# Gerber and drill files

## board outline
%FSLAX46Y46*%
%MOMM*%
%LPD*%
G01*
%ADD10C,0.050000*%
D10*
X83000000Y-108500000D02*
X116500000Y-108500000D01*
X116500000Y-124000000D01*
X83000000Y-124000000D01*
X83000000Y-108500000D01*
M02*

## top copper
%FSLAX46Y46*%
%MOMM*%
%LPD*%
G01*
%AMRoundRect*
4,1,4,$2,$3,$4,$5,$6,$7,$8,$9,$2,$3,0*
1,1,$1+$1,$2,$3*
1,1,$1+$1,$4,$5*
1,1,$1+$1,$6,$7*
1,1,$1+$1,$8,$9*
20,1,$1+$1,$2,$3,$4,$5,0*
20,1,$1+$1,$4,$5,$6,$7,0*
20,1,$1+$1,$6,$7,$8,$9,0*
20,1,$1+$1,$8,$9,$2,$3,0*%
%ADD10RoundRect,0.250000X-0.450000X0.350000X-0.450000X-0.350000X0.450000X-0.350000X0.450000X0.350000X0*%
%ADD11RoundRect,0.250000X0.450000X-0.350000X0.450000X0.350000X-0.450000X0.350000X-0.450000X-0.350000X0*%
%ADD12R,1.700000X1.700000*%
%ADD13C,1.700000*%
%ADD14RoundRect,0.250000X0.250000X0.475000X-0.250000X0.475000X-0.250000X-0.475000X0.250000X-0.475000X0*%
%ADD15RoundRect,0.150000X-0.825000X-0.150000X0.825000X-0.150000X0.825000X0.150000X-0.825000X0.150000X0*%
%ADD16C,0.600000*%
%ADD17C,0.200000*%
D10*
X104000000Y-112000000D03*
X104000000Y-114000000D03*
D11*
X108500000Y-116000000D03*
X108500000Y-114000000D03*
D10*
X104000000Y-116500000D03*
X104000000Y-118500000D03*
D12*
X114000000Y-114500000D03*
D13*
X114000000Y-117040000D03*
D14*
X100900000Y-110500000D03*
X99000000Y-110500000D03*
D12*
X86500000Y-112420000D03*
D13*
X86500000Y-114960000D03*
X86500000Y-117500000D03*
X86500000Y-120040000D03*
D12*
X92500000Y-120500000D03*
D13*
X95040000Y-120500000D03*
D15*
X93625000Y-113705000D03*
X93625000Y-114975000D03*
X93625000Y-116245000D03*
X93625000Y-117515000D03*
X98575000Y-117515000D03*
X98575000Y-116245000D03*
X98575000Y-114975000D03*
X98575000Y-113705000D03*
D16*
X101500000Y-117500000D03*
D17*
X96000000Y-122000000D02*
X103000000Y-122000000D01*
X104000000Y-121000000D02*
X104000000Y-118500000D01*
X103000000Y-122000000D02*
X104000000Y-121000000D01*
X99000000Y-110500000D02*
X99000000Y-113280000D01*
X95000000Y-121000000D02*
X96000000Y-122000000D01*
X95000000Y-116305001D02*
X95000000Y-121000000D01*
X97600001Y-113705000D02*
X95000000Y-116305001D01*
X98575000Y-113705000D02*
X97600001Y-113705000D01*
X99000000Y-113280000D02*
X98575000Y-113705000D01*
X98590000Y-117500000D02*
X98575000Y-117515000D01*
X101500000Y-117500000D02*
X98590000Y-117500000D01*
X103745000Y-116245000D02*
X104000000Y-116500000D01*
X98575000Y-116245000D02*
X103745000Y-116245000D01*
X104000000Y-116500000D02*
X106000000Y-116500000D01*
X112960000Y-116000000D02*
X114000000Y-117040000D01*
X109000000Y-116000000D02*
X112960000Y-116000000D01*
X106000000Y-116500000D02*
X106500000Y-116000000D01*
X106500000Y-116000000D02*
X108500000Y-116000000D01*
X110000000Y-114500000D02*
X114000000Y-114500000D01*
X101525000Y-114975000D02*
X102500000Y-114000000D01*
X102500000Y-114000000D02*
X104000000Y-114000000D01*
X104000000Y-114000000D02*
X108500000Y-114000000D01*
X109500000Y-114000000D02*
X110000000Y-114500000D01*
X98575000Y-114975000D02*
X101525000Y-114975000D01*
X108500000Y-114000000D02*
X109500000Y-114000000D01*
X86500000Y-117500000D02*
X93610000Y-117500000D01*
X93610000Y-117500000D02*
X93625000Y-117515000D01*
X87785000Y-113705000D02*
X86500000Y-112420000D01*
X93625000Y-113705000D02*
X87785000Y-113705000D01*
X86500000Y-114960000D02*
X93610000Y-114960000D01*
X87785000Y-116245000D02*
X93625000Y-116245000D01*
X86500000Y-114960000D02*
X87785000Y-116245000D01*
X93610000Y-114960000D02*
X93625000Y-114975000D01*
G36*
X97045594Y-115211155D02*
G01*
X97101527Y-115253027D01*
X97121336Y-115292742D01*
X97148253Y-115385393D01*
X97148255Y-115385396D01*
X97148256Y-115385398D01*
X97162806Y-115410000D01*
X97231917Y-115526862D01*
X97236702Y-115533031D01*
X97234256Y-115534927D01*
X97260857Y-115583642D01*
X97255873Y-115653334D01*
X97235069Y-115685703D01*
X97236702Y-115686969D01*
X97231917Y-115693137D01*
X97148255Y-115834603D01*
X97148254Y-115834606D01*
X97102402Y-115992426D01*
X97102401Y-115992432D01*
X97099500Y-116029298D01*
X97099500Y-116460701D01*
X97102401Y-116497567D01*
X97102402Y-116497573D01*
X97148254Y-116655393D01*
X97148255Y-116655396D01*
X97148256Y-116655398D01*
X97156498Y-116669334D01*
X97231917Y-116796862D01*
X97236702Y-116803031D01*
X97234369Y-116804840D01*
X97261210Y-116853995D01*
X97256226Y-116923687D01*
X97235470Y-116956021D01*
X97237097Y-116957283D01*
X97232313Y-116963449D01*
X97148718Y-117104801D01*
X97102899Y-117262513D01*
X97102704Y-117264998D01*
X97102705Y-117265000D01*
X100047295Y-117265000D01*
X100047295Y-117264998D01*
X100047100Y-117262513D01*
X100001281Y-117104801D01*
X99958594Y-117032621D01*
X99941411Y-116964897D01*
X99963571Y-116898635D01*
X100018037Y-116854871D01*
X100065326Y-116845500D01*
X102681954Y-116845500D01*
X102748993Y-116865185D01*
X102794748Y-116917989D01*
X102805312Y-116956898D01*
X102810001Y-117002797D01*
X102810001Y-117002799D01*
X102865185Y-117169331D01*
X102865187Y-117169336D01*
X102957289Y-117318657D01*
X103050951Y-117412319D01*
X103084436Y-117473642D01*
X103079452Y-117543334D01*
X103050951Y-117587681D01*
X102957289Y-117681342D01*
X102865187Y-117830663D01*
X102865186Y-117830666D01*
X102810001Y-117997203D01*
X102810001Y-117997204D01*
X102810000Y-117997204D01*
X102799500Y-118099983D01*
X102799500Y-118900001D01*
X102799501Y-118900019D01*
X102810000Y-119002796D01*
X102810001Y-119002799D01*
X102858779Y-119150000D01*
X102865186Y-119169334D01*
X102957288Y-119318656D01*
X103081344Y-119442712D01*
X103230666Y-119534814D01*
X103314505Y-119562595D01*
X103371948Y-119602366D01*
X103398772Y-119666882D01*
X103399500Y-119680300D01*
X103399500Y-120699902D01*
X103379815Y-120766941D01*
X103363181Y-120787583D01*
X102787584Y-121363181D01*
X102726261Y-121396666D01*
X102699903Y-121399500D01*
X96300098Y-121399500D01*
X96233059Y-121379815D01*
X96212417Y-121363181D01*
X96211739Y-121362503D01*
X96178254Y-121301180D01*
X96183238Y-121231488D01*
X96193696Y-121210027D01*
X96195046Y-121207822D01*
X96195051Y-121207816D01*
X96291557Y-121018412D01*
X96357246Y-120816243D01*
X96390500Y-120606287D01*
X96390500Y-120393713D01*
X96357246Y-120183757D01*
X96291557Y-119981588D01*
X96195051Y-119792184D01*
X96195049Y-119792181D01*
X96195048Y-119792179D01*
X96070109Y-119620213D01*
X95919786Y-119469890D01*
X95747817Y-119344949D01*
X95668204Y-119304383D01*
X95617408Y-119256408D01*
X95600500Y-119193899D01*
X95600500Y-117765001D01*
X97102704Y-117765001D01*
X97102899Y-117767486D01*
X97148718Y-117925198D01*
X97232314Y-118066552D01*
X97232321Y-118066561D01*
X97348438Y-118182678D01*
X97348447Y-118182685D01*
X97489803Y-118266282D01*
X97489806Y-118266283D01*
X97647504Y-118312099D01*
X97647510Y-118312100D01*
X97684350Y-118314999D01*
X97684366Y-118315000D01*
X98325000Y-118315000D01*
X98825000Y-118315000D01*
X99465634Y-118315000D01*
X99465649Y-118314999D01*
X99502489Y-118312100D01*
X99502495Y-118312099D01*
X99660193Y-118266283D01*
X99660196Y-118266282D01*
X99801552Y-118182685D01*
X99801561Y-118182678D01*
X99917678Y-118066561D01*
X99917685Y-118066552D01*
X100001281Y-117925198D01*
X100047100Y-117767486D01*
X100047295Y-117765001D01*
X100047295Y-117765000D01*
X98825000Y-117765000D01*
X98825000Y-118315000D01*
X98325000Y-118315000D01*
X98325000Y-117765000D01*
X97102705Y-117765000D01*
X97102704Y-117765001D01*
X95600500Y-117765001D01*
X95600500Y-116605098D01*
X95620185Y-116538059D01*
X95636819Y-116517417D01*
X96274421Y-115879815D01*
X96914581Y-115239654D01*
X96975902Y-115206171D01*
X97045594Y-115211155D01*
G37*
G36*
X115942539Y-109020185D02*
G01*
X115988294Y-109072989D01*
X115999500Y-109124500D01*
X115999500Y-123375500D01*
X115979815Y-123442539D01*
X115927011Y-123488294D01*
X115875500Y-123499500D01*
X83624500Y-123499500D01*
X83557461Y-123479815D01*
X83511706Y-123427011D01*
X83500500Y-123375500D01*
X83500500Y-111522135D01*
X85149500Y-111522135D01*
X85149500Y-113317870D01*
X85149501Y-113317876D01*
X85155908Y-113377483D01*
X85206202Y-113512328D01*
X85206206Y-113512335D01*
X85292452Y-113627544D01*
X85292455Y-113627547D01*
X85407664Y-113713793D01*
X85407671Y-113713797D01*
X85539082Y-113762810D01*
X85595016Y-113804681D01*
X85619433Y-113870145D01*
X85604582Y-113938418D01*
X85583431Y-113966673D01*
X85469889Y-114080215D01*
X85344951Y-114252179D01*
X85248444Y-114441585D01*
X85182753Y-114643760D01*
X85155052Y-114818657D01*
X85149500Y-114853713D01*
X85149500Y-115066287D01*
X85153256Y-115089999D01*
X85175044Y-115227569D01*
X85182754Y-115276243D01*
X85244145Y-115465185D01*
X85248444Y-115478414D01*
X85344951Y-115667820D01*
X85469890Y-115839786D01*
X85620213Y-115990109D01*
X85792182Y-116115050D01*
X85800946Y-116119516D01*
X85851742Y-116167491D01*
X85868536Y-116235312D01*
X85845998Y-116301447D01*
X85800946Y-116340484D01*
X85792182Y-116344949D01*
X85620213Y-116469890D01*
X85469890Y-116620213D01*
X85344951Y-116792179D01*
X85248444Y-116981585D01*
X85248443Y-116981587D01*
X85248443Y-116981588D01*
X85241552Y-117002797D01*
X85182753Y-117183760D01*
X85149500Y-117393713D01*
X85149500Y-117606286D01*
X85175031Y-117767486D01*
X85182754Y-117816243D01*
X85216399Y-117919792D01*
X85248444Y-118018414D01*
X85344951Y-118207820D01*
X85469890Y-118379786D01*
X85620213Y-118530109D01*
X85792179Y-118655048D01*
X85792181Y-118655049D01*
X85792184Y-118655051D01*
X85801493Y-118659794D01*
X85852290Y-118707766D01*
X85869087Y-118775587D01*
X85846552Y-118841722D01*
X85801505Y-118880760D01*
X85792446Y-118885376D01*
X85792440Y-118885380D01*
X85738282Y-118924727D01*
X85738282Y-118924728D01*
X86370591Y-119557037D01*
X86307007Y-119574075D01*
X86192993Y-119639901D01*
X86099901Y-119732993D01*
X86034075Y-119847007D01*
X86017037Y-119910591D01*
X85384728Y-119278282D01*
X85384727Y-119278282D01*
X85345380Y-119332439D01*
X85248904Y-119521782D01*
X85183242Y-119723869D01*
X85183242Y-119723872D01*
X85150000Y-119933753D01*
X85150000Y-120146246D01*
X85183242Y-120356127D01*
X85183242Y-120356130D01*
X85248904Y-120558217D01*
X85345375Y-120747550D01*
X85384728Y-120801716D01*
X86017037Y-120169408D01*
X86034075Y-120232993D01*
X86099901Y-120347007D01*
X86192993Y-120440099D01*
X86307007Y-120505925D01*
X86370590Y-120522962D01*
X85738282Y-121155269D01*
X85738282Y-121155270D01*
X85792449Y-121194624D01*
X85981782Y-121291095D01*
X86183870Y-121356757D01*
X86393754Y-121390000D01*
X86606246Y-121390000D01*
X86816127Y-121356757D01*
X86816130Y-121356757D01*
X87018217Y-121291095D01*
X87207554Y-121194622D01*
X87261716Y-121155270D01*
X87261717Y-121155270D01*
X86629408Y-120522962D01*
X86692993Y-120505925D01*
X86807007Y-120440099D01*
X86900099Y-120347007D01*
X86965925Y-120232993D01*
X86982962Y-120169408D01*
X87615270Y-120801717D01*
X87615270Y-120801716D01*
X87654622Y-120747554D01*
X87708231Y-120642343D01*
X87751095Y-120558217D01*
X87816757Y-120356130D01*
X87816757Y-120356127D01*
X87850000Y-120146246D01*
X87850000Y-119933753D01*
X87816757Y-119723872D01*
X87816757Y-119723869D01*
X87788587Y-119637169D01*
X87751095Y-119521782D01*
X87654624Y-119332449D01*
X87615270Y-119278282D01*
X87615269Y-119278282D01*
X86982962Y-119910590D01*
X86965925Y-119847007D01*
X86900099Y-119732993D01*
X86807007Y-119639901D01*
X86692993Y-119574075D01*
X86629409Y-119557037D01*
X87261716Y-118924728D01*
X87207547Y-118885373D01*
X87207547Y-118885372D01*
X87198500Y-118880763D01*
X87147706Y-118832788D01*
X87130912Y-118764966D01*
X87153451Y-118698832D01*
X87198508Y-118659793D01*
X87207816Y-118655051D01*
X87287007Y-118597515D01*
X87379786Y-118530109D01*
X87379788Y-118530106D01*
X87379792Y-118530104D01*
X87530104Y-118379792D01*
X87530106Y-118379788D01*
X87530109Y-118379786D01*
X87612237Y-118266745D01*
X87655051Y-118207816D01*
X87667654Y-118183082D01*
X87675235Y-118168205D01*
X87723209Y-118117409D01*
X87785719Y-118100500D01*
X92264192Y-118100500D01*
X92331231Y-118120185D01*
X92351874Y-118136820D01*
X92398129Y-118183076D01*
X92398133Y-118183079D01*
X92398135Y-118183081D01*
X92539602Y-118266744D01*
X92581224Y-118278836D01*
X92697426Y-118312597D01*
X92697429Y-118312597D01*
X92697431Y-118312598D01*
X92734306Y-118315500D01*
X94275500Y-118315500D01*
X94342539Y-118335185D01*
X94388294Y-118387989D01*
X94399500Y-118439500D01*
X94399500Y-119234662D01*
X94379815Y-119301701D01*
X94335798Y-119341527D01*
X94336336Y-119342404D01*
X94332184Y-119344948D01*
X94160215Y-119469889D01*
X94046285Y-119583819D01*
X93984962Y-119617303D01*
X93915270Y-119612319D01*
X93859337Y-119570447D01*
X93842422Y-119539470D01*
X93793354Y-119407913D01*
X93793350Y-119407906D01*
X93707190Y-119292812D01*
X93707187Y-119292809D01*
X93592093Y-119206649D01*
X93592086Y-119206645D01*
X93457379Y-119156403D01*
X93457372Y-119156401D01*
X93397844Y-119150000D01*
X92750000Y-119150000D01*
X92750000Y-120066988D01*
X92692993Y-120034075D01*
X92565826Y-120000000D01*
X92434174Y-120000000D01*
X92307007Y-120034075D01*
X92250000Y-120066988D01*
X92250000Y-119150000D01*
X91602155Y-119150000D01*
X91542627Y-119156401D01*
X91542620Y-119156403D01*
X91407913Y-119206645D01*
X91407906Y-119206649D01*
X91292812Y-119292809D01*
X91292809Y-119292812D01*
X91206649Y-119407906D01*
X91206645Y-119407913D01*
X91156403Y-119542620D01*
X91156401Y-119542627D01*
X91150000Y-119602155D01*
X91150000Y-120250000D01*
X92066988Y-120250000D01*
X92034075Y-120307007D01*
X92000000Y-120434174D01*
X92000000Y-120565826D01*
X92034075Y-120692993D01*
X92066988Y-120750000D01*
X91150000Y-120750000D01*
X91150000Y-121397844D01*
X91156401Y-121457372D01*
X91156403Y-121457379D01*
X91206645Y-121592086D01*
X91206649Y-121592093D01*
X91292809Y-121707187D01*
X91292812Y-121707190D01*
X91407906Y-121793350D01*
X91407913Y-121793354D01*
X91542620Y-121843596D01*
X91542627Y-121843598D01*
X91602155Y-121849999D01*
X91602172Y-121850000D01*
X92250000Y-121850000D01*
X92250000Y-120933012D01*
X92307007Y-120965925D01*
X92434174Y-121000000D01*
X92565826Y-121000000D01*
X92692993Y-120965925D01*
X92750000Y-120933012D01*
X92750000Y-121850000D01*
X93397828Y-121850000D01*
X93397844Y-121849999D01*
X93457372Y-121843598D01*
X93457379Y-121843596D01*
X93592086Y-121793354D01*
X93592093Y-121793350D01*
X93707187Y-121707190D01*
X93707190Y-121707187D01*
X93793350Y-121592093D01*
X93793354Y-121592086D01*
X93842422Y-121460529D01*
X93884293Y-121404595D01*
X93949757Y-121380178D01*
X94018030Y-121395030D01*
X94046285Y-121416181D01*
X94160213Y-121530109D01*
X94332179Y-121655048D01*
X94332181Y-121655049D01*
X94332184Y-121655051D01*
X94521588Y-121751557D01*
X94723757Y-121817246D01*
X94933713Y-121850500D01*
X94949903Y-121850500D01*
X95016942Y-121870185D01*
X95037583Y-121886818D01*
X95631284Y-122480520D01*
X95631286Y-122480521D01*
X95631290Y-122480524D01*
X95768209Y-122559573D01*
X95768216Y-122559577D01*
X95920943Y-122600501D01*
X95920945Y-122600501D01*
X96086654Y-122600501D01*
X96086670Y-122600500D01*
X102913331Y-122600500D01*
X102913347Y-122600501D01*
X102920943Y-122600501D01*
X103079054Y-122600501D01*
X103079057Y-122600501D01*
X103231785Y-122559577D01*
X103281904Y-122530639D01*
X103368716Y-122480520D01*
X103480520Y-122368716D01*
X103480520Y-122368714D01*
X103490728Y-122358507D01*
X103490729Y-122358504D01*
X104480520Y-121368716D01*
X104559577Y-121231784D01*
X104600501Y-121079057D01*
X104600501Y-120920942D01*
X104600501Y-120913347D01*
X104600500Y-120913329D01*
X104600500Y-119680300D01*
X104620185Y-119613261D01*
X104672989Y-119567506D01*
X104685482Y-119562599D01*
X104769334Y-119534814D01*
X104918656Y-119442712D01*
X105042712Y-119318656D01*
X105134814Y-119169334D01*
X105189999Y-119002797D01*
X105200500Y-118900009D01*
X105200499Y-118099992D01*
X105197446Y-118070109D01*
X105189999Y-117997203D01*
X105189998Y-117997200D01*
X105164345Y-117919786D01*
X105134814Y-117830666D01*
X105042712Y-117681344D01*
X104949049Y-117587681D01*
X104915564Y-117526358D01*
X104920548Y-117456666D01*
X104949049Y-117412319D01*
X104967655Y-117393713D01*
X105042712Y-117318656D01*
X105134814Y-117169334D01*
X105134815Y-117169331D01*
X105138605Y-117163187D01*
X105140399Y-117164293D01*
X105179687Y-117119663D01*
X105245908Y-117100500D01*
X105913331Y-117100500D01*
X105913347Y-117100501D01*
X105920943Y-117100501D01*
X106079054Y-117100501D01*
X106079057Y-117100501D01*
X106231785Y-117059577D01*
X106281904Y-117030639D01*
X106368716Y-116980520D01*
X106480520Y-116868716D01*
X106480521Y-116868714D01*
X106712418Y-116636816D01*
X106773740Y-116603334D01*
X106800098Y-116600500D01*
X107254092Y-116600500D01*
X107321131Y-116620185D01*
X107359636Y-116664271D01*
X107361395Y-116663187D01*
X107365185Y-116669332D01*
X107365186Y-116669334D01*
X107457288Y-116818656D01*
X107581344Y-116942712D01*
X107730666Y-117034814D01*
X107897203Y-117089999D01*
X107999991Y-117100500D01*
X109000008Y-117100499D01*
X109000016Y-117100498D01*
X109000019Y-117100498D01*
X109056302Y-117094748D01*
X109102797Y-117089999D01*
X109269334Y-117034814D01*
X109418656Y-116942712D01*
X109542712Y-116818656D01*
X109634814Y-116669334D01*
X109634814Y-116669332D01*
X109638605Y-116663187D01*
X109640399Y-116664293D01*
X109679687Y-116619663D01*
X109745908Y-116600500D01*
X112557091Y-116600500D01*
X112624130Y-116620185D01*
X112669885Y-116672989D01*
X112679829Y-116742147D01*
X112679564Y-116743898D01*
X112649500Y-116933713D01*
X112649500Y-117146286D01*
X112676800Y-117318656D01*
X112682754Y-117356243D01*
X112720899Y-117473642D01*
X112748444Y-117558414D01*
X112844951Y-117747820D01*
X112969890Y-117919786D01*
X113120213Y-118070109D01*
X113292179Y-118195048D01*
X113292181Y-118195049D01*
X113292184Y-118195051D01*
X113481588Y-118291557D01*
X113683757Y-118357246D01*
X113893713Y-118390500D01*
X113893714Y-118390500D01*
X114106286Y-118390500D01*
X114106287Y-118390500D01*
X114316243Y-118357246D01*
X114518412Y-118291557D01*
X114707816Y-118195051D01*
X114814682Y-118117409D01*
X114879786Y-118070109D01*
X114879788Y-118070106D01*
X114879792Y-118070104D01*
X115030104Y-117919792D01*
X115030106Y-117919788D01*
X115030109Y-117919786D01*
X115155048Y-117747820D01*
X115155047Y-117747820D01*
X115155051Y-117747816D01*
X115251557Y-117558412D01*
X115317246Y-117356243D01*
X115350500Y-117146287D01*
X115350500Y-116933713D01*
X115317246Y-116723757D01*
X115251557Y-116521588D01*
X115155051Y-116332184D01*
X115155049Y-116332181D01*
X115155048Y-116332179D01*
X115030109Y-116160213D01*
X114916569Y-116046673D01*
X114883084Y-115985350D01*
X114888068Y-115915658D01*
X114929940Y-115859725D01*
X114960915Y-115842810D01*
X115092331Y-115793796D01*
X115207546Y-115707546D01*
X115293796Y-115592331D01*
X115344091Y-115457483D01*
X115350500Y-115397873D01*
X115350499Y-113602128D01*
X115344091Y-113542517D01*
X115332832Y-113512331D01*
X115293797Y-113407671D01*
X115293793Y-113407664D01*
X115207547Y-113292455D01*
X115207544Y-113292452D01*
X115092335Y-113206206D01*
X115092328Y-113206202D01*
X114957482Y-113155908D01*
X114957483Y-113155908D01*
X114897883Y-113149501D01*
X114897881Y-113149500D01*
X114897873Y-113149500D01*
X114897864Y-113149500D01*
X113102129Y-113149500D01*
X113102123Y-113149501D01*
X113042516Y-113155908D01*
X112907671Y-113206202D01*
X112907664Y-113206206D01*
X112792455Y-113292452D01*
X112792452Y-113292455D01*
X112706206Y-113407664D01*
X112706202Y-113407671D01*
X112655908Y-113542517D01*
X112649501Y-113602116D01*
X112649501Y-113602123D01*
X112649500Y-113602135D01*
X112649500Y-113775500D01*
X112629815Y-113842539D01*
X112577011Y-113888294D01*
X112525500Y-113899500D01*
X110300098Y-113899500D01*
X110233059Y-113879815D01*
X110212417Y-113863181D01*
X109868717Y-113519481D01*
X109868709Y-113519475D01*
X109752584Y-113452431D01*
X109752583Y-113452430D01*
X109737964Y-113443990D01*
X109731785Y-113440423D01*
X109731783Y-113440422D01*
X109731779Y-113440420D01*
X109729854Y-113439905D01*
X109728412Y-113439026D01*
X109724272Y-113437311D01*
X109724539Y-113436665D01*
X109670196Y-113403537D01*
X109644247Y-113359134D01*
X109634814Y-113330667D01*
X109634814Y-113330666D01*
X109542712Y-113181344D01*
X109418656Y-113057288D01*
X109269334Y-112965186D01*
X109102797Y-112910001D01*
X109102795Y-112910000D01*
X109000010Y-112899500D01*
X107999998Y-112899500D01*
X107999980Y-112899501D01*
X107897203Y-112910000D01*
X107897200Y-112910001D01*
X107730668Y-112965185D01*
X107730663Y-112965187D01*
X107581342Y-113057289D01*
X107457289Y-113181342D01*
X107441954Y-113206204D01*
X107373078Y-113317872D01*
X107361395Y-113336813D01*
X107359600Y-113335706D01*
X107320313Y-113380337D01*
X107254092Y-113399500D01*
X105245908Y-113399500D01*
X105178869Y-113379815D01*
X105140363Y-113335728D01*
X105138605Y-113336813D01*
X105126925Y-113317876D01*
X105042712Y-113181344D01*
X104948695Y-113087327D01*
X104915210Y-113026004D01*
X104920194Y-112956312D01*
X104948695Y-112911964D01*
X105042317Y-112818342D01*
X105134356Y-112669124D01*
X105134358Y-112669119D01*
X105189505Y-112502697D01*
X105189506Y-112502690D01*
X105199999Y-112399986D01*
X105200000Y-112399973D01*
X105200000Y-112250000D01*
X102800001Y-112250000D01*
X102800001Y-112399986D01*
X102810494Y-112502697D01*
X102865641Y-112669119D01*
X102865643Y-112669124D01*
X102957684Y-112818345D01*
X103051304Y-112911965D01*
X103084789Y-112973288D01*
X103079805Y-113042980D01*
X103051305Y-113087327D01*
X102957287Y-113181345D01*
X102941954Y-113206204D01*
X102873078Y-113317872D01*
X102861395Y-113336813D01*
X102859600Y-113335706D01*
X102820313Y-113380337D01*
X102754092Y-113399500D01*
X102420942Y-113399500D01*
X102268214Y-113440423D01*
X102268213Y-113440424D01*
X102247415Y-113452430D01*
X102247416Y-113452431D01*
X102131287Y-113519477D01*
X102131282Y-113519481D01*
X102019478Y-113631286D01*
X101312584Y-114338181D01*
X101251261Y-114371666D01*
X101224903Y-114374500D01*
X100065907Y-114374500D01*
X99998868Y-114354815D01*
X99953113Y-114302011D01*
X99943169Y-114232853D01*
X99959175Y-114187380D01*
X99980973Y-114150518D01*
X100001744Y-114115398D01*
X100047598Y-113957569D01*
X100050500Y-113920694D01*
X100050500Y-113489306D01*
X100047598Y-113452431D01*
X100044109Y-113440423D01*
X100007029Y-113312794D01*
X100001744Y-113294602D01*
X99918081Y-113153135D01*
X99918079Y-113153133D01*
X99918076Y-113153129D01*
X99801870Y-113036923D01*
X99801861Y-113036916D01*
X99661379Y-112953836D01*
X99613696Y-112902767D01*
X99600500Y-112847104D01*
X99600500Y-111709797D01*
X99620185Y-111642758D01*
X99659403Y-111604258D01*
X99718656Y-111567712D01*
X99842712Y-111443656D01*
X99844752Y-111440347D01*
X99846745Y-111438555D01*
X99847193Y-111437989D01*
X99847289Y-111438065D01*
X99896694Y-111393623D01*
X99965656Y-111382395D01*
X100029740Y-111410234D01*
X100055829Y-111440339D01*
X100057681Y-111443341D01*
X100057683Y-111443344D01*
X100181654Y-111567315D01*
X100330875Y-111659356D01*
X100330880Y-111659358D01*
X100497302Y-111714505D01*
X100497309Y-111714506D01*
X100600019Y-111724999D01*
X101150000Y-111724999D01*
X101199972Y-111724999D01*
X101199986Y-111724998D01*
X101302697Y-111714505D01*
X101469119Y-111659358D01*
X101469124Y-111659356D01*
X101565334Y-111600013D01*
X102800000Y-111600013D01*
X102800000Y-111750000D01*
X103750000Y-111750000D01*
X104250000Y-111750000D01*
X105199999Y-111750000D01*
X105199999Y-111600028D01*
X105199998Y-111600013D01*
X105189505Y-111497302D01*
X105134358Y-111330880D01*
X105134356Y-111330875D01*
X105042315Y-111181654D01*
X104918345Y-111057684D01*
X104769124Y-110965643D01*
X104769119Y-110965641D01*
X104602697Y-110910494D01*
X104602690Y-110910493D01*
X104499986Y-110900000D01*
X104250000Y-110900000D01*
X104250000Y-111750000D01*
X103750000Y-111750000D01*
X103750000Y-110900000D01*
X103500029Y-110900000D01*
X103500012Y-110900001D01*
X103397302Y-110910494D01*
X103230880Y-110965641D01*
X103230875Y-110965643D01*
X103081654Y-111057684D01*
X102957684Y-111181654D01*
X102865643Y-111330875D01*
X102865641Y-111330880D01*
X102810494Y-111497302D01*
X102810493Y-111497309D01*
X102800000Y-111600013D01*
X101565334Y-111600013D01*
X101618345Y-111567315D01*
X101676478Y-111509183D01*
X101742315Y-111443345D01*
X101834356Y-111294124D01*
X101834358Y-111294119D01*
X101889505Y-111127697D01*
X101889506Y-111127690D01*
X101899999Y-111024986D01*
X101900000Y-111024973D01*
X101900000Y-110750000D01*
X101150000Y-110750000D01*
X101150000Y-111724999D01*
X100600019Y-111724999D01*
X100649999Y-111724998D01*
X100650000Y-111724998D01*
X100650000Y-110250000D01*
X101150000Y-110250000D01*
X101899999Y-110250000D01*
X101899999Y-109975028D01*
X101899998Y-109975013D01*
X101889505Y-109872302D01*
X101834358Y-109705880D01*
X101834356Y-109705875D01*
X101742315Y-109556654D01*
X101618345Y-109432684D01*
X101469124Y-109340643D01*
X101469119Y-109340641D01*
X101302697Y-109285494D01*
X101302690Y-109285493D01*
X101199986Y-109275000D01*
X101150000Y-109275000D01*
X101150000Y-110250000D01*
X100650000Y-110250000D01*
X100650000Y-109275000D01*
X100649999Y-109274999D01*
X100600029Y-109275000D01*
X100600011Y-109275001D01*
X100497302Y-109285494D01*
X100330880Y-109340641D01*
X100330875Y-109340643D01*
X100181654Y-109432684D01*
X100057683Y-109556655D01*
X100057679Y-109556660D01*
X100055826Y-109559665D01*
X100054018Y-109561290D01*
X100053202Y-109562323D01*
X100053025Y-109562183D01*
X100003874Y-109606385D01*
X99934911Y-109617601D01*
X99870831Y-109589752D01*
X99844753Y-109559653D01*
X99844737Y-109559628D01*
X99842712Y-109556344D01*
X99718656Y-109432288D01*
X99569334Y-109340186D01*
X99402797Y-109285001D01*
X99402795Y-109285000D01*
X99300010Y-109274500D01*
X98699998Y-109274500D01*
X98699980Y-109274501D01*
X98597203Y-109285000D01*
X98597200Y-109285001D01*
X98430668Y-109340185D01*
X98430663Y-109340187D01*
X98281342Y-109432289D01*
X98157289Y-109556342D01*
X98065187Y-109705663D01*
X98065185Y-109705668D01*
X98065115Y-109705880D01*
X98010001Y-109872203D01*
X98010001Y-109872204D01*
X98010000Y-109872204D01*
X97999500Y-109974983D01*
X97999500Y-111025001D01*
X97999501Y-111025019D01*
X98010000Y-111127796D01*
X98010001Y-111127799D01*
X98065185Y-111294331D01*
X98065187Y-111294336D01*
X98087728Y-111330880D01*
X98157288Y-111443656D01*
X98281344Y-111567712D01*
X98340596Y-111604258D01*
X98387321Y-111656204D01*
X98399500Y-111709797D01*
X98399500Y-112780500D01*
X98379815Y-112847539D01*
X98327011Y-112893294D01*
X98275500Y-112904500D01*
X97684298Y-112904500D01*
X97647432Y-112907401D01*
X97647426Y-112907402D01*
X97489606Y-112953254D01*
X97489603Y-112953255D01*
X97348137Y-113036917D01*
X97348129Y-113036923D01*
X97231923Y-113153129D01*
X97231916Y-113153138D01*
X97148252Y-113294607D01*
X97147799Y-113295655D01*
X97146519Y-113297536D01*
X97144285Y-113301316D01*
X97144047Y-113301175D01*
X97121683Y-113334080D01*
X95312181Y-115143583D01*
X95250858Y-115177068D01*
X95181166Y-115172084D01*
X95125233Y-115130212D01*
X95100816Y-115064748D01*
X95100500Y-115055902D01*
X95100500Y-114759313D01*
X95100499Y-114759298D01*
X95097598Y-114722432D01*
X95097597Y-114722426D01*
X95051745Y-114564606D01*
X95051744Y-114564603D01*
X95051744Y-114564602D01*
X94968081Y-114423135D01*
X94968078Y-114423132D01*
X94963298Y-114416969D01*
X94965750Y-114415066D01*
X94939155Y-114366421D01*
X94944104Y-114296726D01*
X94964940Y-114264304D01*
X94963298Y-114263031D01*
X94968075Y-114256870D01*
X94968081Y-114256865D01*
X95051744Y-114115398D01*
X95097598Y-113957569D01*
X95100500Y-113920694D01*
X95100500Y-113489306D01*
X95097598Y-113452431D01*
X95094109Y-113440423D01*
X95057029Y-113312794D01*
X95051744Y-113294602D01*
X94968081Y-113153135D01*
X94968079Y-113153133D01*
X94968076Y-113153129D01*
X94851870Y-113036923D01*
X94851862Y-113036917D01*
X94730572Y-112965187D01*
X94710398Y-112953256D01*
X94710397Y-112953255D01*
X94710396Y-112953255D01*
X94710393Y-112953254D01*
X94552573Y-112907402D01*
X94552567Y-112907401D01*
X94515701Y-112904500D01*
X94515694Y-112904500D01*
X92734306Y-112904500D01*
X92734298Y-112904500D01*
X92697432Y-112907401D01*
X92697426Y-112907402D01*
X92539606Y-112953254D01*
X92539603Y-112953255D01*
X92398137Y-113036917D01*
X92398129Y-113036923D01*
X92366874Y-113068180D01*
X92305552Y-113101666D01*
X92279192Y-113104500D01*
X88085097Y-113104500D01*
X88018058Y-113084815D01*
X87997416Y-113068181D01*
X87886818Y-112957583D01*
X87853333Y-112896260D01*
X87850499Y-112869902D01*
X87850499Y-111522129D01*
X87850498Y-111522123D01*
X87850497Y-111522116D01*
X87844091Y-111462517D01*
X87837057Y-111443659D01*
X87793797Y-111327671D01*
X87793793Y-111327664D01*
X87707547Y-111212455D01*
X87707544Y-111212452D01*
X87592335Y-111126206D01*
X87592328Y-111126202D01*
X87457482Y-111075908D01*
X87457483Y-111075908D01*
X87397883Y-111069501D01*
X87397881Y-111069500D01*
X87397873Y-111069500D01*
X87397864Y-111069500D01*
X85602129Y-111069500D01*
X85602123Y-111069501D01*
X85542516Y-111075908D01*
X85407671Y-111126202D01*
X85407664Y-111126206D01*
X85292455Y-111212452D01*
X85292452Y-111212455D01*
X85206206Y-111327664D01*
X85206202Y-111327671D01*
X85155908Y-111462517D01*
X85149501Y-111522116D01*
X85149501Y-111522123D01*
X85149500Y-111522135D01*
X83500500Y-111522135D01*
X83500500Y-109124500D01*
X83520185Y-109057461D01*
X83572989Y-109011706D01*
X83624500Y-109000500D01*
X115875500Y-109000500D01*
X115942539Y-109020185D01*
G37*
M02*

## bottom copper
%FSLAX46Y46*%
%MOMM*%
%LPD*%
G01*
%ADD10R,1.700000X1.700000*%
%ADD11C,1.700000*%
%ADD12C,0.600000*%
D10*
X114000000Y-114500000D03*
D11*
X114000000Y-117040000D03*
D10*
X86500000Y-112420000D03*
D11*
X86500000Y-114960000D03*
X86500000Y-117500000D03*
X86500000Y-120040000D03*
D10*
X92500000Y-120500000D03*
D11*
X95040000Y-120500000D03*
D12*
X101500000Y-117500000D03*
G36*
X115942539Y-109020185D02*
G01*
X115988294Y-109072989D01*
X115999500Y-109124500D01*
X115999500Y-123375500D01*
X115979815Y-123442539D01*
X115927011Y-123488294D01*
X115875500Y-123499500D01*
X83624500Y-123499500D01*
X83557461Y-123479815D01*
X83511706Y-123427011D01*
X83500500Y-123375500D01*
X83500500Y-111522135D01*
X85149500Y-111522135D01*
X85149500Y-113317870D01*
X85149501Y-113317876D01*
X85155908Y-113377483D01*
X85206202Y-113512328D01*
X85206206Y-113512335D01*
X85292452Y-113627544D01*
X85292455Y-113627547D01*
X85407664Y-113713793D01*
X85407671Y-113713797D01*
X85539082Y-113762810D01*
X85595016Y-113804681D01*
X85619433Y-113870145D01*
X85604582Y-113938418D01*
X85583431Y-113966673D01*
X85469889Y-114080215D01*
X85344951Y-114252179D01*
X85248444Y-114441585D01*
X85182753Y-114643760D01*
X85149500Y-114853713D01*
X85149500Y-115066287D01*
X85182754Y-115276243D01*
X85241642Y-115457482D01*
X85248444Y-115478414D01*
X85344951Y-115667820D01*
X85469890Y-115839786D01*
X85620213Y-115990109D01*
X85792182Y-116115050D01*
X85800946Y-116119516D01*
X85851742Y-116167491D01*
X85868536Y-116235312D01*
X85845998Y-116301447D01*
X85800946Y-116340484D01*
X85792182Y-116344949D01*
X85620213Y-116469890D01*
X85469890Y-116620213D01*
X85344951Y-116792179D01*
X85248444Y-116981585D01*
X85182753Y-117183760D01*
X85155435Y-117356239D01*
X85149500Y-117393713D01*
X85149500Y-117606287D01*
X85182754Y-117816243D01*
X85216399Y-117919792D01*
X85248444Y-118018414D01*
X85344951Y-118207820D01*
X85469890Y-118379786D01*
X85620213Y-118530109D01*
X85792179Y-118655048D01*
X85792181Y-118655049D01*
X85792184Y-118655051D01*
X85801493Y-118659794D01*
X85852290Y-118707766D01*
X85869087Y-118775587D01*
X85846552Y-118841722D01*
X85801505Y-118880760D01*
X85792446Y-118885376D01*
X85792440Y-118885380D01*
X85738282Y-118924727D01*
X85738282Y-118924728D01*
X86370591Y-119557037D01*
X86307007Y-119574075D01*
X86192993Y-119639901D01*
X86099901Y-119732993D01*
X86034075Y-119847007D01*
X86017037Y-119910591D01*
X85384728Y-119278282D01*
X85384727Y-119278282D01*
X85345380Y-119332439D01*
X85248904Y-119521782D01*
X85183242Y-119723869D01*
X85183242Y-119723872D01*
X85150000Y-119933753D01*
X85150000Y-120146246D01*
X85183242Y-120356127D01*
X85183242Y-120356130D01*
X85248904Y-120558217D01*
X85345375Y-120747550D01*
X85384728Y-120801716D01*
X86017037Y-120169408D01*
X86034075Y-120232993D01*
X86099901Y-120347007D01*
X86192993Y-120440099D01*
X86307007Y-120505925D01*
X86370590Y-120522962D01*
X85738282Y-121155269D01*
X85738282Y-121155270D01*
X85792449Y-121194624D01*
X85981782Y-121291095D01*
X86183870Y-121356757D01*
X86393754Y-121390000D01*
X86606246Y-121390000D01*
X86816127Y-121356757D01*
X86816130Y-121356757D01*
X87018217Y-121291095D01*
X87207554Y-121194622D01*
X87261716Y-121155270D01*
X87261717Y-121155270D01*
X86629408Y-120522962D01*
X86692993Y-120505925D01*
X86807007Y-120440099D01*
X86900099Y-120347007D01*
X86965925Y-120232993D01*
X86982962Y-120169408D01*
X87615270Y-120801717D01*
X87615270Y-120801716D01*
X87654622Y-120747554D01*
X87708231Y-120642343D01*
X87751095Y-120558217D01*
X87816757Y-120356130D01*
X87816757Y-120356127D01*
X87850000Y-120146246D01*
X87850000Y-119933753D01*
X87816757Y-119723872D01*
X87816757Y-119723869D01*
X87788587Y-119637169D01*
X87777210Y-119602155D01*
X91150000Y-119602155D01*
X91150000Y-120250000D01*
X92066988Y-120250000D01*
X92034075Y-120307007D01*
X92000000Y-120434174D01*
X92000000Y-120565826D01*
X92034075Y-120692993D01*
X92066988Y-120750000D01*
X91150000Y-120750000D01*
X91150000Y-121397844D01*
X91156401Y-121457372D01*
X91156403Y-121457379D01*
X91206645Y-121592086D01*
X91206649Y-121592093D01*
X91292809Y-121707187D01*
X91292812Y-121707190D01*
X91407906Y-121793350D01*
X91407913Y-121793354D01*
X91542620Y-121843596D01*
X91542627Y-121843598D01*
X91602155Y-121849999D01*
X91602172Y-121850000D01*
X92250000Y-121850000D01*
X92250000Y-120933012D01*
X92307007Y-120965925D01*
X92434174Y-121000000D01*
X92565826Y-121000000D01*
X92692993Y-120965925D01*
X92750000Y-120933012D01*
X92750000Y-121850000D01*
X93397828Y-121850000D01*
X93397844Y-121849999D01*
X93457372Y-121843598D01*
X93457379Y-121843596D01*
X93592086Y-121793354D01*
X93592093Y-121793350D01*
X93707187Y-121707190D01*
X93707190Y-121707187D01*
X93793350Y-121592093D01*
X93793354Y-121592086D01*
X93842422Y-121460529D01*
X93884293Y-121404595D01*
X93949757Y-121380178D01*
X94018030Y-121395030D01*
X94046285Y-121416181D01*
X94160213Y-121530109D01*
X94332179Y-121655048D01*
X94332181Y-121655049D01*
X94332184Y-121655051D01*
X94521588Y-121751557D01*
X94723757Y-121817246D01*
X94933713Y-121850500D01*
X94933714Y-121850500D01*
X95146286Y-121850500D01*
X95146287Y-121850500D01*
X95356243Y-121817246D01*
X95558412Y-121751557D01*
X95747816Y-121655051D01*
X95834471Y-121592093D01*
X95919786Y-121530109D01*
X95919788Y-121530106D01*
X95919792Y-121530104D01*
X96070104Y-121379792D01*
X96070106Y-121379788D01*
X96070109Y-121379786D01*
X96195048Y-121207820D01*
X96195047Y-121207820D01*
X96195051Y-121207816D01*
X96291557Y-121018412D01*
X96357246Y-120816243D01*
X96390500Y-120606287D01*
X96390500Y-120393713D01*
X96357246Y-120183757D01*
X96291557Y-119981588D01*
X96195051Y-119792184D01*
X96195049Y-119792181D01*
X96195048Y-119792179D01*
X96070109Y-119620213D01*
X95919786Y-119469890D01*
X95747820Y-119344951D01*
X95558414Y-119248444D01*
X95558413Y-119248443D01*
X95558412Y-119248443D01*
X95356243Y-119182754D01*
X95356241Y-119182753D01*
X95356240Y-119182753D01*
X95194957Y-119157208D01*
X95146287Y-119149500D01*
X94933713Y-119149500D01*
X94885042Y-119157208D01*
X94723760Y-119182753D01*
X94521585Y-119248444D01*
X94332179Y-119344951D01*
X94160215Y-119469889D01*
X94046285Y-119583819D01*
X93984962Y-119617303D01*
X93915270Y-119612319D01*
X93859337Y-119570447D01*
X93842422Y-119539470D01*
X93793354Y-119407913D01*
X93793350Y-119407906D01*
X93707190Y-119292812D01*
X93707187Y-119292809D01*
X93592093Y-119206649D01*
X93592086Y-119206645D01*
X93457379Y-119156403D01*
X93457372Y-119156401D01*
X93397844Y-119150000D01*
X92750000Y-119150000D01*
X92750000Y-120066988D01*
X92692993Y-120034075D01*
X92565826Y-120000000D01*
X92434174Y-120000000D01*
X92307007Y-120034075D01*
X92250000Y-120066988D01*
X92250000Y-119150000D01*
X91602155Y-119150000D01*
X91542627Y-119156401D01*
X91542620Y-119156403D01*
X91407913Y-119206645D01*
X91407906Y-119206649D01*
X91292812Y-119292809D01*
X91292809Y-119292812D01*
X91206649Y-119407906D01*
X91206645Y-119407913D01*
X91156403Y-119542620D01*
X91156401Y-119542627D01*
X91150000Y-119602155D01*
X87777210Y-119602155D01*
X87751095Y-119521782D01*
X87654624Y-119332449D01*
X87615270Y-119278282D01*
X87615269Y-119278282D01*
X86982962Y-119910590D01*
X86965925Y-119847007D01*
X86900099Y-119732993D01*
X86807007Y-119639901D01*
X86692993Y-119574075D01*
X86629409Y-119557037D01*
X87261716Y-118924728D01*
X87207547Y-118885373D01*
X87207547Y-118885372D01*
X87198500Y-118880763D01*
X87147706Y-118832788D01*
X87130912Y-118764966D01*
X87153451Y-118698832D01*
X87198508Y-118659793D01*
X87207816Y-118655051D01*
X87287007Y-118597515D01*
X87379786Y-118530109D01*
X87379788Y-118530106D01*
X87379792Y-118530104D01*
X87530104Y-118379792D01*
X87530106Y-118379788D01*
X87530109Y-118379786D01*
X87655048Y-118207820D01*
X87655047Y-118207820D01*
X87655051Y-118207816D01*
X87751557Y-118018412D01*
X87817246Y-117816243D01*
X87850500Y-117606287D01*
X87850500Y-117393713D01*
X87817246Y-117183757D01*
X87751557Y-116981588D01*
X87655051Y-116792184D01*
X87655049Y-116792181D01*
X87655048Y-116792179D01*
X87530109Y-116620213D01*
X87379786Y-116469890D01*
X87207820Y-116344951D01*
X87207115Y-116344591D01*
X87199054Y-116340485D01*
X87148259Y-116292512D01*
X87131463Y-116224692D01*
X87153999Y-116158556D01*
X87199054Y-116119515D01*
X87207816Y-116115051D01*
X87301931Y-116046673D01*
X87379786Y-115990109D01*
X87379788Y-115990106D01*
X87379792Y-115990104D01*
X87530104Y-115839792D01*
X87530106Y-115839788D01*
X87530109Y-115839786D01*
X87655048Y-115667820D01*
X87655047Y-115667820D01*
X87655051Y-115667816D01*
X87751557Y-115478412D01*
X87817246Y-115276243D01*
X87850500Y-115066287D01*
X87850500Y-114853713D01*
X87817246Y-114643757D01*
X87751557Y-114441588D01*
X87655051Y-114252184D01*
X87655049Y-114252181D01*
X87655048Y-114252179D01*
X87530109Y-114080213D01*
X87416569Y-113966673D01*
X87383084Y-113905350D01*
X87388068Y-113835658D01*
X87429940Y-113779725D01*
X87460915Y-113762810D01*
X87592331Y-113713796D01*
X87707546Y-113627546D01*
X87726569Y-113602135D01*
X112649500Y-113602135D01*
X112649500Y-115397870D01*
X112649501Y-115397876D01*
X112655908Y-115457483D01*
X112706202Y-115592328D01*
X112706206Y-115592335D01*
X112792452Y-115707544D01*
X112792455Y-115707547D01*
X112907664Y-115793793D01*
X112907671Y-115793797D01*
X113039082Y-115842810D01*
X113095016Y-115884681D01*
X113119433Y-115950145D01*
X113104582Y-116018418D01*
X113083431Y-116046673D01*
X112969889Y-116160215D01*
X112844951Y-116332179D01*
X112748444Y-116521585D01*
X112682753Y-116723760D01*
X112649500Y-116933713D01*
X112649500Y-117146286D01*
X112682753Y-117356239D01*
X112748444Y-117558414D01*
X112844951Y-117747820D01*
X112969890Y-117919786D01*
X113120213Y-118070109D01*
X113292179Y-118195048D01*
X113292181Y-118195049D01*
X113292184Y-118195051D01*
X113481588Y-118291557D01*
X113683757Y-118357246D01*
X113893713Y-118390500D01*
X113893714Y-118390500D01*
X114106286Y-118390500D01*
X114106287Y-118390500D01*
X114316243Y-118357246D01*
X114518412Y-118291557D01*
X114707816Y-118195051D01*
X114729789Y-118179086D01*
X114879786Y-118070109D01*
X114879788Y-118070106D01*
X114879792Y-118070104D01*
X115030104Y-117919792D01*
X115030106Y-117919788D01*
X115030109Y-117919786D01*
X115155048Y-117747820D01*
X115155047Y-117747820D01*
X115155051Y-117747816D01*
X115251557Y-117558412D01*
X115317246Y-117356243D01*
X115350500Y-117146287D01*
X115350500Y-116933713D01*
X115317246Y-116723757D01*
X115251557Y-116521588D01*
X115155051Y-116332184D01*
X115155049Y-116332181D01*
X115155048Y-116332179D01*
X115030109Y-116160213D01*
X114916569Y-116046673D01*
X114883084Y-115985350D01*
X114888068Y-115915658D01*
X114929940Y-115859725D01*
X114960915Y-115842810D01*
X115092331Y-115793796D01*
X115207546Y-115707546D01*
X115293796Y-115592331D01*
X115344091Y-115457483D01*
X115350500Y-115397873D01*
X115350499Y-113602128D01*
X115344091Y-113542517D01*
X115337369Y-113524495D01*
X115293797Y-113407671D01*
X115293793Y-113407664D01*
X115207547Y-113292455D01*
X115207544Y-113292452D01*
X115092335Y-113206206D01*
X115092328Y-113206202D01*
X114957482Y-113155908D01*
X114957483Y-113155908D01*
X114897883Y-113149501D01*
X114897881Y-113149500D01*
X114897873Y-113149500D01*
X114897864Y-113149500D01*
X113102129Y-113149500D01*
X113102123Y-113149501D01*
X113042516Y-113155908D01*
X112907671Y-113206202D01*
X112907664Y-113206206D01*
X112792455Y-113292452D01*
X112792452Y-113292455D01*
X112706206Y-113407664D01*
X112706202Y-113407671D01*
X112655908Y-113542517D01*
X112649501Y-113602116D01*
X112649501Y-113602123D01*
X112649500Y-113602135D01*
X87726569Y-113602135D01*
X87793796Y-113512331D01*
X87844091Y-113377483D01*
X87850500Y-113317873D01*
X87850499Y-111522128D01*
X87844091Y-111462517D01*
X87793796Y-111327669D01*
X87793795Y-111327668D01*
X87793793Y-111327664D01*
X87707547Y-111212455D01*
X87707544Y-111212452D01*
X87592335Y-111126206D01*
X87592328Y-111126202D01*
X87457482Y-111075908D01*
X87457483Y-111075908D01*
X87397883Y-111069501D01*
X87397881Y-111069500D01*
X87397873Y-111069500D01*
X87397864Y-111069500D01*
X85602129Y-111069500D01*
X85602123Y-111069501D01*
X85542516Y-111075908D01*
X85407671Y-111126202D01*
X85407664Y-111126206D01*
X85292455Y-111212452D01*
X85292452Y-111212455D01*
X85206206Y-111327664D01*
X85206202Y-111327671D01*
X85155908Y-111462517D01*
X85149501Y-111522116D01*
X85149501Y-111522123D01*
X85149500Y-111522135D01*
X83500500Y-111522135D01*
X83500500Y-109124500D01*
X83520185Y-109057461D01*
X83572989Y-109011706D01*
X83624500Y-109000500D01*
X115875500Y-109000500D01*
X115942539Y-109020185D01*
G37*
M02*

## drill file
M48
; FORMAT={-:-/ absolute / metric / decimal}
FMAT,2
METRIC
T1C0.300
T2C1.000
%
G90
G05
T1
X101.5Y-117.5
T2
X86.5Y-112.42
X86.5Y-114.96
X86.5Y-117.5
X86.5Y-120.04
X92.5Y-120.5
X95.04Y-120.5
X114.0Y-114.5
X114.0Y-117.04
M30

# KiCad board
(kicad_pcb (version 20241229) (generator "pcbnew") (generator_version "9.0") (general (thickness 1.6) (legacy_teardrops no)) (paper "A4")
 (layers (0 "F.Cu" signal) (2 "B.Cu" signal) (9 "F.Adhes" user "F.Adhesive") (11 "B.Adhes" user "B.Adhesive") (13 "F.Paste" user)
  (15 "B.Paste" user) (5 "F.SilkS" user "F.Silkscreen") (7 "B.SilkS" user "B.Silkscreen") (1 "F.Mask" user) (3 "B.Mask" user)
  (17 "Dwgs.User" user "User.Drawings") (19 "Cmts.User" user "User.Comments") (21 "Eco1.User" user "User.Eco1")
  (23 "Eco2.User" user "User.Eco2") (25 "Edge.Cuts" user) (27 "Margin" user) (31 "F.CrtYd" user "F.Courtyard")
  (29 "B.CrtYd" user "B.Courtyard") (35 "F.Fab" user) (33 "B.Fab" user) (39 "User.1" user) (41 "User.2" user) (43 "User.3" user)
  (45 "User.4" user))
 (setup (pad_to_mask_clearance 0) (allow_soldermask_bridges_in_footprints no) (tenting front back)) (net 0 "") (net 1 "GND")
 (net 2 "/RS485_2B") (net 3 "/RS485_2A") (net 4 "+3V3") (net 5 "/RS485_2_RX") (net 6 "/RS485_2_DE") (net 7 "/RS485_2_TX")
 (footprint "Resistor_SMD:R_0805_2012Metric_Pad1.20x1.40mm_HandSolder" (layer "F.Cu") (at 104 113 -90)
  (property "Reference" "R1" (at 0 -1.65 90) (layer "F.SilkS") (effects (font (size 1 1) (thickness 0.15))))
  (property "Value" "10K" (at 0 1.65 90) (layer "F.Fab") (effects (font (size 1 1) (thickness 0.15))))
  (pad "1" smd roundrect (at -1 0 270) (size 1.2 1.4) (layers "F.Cu" "F.Mask" "F.Paste") (roundrect_rratio 0.208333) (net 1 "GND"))
  (pad "2" smd roundrect (at 1 0 270) (size 1.2 1.4) (layers "F.Cu" "F.Mask" "F.Paste") (roundrect_rratio 0.208333) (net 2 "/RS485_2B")))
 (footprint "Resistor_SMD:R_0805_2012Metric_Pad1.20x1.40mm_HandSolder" (layer "F.Cu") (at 108.5 115 90)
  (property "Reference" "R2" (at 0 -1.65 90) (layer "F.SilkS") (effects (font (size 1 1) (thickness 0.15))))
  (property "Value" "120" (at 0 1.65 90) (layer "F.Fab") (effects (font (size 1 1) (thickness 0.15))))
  (pad "1" smd roundrect (at -1 0 90) (size 1.2 1.4) (layers "F.Cu" "F.Mask" "F.Paste") (roundrect_rratio 0.208333) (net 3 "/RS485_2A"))
  (pad "2" smd roundrect (at 1 0 90) (size 1.2 1.4) (layers "F.Cu" "F.Mask" "F.Paste") (roundrect_rratio 0.208333) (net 2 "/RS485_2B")))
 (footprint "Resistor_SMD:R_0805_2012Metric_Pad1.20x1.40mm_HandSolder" (layer "F.Cu") (at 104 117.5 -90)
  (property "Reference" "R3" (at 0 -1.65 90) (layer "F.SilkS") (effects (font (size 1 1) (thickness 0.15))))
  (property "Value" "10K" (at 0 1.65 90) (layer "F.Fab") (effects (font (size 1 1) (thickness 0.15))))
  (pad "1" smd roundrect (at -1 0 270) (size 1.2 1.4) (layers "F.Cu" "F.Mask" "F.Paste") (roundrect_rratio 0.208333) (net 3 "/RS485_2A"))
  (pad "2" smd roundrect (at 1 0 270) (size 1.2 1.4) (layers "F.Cu" "F.Mask" "F.Paste") (roundrect_rratio 0.208333) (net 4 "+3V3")))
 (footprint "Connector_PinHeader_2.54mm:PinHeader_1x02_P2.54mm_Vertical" (layer "F.Cu") (at 114 114.5)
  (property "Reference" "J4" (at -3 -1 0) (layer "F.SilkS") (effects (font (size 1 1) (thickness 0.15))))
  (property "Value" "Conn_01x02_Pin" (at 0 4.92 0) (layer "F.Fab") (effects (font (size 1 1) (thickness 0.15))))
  (pad "1" thru_hole rect (at 0 0) (size 1.7 1.7) (drill 1) (layers "*.Cu" "*.Mask") (remove_unused_layers no) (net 2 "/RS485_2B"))
  (pad "2" thru_hole circle (at 0 2.54) (size 1.7 1.7) (drill 1) (layers "*.Cu" "*.Mask") (remove_unused_layers no) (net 3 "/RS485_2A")))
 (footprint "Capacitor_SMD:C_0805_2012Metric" (layer "F.Cu") (at 99.95 110.5 180)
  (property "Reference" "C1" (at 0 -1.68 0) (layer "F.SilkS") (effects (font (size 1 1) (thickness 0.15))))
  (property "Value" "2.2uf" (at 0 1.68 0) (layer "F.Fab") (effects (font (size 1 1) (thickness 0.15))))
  (pad "1" smd roundrect (at -0.95 0 180) (size 1 1.45) (layers "F.Cu" "F.Mask" "F.Paste") (roundrect_rratio 0.25) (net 1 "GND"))
  (pad "2" smd roundrect (at 0.95 0 180) (size 1 1.45) (layers "F.Cu" "F.Mask" "F.Paste") (roundrect_rratio 0.25) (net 4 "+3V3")))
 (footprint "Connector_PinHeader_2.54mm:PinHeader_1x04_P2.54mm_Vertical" (layer "F.Cu") (at 86.5 112.42)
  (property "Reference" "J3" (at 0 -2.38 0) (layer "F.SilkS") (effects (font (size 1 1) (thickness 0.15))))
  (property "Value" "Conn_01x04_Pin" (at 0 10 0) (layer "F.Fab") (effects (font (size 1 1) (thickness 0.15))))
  (pad "1" thru_hole rect (at 0 0) (size 1.7 1.7) (drill 1) (layers "*.Cu" "*.Mask") (remove_unused_layers no) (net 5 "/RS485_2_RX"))
  (pad "2" thru_hole circle (at 0 2.54) (size 1.7 1.7) (drill 1) (layers "*.Cu" "*.Mask") (remove_unused_layers no) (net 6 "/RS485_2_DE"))
  (pad "3" thru_hole circle (at 0 5.08) (size 1.7 1.7) (drill 1) (layers "*.Cu" "*.Mask") (remove_unused_layers no) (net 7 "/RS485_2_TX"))
  (pad "4" thru_hole circle (at 0 7.62) (size 1.7 1.7) (drill 1) (layers "*.Cu" "*.Mask") (remove_unused_layers no) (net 1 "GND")))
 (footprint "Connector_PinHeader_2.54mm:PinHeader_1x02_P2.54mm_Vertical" (layer "F.Cu") (at 92.5 120.5 90)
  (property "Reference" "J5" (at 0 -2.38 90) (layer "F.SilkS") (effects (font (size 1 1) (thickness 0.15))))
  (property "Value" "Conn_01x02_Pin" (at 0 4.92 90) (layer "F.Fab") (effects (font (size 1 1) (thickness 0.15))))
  (pad "1" thru_hole rect (at 0 0 90) (size 1.7 1.7) (drill 1) (layers "*.Cu" "*.Mask") (remove_unused_layers no) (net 1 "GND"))
  (pad "2" thru_hole circle (at 0 2.54 90) (size 1.7 1.7) (drill 1) (layers "*.Cu" "*.Mask") (remove_unused_layers no) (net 4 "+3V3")))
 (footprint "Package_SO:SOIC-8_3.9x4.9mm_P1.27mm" (layer "F.Cu") (at 96.1 115.61)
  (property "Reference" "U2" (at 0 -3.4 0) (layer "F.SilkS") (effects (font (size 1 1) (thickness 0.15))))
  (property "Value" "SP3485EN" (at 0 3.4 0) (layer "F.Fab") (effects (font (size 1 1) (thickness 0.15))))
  (pad "1" smd roundrect (at -2.475 -1.905) (size 1.95 0.6) (layers "F.Cu" "F.Mask" "F.Paste") (roundrect_rratio 0.25) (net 5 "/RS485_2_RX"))
  (pad "2" smd roundrect (at -2.475 -0.635) (size 1.95 0.6) (layers "F.Cu" "F.Mask" "F.Paste") (roundrect_rratio 0.25) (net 6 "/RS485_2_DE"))
  (pad "3" smd roundrect (at -2.475 0.635) (size 1.95 0.6) (layers "F.Cu" "F.Mask" "F.Paste") (roundrect_rratio 0.25) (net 6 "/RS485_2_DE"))
  (pad "4" smd roundrect (at -2.475 1.905) (size 1.95 0.6) (layers "F.Cu" "F.Mask" "F.Paste") (roundrect_rratio 0.25) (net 7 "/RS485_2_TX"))
  (pad "5" smd roundrect (at 2.475 1.905) (size 1.95 0.6) (layers "F.Cu" "F.Mask" "F.Paste") (roundrect_rratio 0.25) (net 1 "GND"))
  (pad "6" smd roundrect (at 2.475 0.635) (size 1.95 0.6) (layers "F.Cu" "F.Mask" "F.Paste") (roundrect_rratio 0.25) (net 3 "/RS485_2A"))
  (pad "7" smd roundrect (at 2.475 -0.635) (size 1.95 0.6) (layers "F.Cu" "F.Mask" "F.Paste") (roundrect_rratio 0.25) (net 2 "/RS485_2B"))
  (pad "8" smd roundrect (at 2.475 -1.905) (size 1.95 0.6) (layers "F.Cu" "F.Mask" "F.Paste") (roundrect_rratio 0.25) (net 4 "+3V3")))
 (gr_rect (start 83 108.5) (end 116.5 124) (stroke (width 0.05) (type default)) (fill no) (layer "Edge.Cuts"))
 (segment (start 96 122) (end 103 122) (width 0.2) (layer "F.Cu") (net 4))
 (segment (start 104 121) (end 104 118.5) (width 0.2) (layer "F.Cu") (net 4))
 (segment (start 103 122) (end 104 121) (width 0.2) (layer "F.Cu") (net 4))
 (segment (start 99 110.5) (end 99 113.28) (width 0.2) (layer "F.Cu") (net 4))
 (segment (start 95 121) (end 96 122) (width 0.2) (layer "F.Cu") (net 4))
 (segment (start 95 116.305001) (end 95 121) (width 0.2) (layer "F.Cu") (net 4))
 (segment (start 97.600001 113.705) (end 95 116.305001) (width 0.2) (layer "F.Cu") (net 4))
 (segment (start 98.575 113.705) (end 97.600001 113.705) (width 0.2) (layer "F.Cu") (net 4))
 (segment (start 99 113.28) (end 98.575 113.705) (width 0.2) (layer "F.Cu") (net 4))
 (segment (start 98.59 117.5) (end 98.575 117.515) (width 0.2) (layer "F.Cu") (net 1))
 (segment (start 101.5 117.5) (end 98.59 117.5) (width 0.2) (layer "F.Cu") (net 1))
 (via (at 101.5 117.5) (size 0.6) (drill 0.3) (layers "F.Cu" "B.Cu") (free yes) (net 1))
 (segment (start 103.745 116.245) (end 104 116.5) (width 0.2) (layer "F.Cu") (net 3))
 (segment (start 98.575 116.245) (end 103.745 116.245) (width 0.2) (layer "F.Cu") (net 3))
 (segment (start 104 116.5) (end 106 116.5) (width 0.2) (layer "F.Cu") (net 3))
 (segment (start 112.96 116) (end 114 117.04) (width 0.2) (layer "F.Cu") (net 3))
 (segment (start 109 116) (end 112.96 116) (width 0.2) (layer "F.Cu") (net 3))
 (segment (start 106 116.5) (end 106.5 116) (width 0.2) (layer "F.Cu") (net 3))
 (segment (start 106.5 116) (end 108.5 116) (width 0.2) (layer "F.Cu") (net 3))
 (segment (start 110 114.5) (end 114 114.5) (width 0.2) (layer "F.Cu") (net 2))
 (segment (start 101.525 114.975) (end 102.5 114) (width 0.2) (layer "F.Cu") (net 2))
 (segment (start 102.5 114) (end 104 114) (width 0.2) (layer "F.Cu") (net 2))
 (segment (start 104 114) (end 108.5 114) (width 0.2) (layer "F.Cu") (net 2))
 (segment (start 109.5 114) (end 110 114.5) (width 0.2) (layer "F.Cu") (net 2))
 (segment (start 98.575 114.975) (end 101.525 114.975) (width 0.2) (layer "F.Cu") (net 2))
 (segment (start 108.5 114) (end 109.5 114) (width 0.2) (layer "F.Cu") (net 2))
 (segment (start 86.5 117.5) (end 93.61 117.5) (width 0.2) (layer "F.Cu") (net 7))
 (segment (start 93.61 117.5) (end 93.625 117.515) (width 0.2) (layer "F.Cu") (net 7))
 (segment (start 87.785 113.705) (end 86.5 112.42) (width 0.2) (layer "F.Cu") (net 5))
 (segment (start 93.625 113.705) (end 87.785 113.705) (width 0.2) (layer "F.Cu") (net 5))
 (segment (start 86.5 114.96) (end 93.61 114.96) (width 0.2) (layer "F.Cu") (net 6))
 (segment (start 87.785 116.245) (end 93.625 116.245) (width 0.2) (layer "F.Cu") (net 6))
 (segment (start 86.5 114.96) (end 87.785 116.245) (width 0.2) (layer "F.Cu") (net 6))
 (segment (start 93.61 114.96) (end 93.625 114.975) (width 0.2) (layer "F.Cu") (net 6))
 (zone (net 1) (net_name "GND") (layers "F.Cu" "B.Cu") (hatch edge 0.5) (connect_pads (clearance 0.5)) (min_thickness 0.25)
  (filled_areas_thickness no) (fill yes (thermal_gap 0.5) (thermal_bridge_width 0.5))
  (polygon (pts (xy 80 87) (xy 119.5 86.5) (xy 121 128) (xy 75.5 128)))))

